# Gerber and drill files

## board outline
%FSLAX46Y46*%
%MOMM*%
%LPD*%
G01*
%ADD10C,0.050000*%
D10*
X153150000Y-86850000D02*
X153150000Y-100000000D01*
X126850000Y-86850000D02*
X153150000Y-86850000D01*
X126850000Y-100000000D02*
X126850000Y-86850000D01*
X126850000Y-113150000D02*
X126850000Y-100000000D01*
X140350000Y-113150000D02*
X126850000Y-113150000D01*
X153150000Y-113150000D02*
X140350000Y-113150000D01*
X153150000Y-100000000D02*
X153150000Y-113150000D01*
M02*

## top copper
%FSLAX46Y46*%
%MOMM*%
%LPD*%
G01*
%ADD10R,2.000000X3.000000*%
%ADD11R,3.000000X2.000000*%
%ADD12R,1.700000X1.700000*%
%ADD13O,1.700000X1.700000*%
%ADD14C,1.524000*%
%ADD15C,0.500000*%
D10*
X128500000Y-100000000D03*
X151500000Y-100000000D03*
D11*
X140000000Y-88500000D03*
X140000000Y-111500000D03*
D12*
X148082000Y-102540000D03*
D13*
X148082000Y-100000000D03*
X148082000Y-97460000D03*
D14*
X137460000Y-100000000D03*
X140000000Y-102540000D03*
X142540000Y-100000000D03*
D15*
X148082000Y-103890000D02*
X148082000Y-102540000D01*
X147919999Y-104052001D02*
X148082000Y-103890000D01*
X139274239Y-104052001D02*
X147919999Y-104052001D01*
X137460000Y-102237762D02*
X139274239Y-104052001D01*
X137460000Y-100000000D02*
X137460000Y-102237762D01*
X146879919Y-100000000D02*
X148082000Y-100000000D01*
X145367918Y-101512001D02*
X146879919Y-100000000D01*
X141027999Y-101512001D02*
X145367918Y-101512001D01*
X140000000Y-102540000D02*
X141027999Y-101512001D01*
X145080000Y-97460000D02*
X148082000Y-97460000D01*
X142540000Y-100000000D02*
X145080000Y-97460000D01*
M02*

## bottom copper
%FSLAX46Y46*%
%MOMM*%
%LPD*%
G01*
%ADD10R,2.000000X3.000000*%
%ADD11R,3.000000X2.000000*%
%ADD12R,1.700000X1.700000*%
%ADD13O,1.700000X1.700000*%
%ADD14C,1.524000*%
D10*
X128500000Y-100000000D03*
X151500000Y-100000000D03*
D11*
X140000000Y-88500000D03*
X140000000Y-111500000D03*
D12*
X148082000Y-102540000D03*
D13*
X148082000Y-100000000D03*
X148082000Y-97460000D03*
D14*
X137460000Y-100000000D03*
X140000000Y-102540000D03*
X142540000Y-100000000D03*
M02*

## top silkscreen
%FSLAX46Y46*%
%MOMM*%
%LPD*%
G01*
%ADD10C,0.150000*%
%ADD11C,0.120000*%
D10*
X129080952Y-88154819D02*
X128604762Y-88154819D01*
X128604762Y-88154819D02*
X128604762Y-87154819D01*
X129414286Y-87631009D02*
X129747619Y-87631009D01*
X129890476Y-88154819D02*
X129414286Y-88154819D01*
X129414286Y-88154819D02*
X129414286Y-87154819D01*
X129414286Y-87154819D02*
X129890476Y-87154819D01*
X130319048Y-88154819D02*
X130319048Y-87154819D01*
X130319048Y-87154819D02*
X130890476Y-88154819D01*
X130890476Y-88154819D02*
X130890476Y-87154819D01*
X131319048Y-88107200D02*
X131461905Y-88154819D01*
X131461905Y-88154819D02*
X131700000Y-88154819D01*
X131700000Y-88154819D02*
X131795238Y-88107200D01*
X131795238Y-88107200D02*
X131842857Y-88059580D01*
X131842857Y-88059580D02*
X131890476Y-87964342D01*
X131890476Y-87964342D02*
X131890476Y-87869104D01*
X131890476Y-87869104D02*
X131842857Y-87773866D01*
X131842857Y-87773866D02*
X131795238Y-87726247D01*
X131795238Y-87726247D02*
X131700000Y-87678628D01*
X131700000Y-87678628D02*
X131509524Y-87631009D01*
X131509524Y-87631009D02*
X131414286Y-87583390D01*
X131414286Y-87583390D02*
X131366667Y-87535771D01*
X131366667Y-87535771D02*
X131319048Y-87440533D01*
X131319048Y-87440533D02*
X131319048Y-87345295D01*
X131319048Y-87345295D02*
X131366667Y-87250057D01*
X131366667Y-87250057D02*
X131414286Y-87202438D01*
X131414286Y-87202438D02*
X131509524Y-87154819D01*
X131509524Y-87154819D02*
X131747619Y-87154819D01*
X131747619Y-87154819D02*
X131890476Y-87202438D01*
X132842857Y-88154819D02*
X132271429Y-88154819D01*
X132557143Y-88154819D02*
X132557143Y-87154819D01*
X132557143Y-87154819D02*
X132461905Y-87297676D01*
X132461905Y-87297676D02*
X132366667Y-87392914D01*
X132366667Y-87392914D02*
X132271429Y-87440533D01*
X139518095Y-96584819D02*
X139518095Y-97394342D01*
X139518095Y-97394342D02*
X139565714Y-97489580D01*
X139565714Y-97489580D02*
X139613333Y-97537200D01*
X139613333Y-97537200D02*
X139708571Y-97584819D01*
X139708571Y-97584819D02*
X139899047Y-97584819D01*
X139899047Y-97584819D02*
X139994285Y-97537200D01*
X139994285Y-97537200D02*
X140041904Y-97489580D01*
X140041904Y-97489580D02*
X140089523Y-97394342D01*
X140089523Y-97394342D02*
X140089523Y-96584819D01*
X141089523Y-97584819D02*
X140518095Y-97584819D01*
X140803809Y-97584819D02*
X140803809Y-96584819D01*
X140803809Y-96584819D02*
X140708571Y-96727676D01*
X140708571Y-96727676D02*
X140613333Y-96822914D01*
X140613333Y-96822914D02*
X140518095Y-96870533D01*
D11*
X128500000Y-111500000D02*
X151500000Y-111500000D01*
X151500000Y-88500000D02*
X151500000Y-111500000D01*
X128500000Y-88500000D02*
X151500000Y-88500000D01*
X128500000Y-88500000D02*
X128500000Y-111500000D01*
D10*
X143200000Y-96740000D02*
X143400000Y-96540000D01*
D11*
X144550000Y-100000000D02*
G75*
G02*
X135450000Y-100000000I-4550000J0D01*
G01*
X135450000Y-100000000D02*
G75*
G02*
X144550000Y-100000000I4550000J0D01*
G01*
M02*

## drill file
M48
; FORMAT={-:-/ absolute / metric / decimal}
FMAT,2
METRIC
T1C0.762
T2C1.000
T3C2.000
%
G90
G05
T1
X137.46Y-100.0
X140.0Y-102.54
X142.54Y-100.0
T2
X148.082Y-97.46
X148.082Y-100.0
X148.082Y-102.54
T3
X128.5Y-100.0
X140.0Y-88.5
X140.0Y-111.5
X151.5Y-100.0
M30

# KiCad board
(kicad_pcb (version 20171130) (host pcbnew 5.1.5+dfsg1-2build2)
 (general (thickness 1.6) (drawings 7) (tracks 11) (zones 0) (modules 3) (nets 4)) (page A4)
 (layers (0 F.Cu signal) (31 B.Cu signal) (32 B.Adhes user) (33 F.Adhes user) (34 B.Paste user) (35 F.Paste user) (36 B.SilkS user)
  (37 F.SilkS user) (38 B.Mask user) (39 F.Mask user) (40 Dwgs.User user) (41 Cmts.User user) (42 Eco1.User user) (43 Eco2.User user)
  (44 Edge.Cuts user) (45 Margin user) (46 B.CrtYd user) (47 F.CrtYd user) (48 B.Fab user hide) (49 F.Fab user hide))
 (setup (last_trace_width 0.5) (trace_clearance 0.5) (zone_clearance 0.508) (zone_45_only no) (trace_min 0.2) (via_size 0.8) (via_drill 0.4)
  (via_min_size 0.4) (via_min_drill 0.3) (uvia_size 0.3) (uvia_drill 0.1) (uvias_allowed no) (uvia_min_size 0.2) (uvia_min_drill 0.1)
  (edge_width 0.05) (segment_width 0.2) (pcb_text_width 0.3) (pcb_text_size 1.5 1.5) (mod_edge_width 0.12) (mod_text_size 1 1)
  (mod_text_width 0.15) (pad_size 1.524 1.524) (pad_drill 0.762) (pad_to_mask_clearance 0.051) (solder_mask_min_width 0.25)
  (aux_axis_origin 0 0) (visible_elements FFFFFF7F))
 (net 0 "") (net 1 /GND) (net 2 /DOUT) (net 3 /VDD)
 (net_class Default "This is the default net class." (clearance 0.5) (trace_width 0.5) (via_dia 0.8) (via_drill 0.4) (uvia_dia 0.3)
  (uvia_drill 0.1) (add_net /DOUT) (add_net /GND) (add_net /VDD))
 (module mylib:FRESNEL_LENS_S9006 (layer F.Cu) (at 140 100)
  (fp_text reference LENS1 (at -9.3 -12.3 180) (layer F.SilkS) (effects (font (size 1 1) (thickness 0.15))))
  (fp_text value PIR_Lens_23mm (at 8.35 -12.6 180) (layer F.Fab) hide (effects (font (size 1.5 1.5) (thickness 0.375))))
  (fp_line (start -11.5 11.5) (end 11.5 11.5) (layer F.SilkS) (width 0.12))
  (fp_line (start 11.5 -11.5) (end 11.5 11.5) (layer F.SilkS) (width 0.12))
  (fp_line (start -11.5 -11.5) (end 11.5 -11.5) (layer F.SilkS) (width 0.12))
  (fp_line (start -11.5 -11.5) (end -11.5 11.5) (layer F.SilkS) (width 0.12))
  (pad "" np_thru_hole rect (at -11.5 0) (size 2 3) (drill 2) (layers *.Cu *.Mask) (clearance 0.5))
  (pad "" np_thru_hole rect (at 11.5 0) (size 2 3) (drill 2) (layers *.Cu *.Mask) (clearance 0.5))
  (pad "" np_thru_hole rect (at 0 -11.5 90) (size 2 3) (drill 2) (layers *.Cu *.Mask) (clearance 0.5))
  (pad "" np_thru_hole rect (at 0 11.5 90) (size 2 3) (drill 2) (layers *.Cu *.Mask) (clearance 0.5)))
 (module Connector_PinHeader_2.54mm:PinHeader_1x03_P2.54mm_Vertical (layer B.Cu) (at 148.082 102.54)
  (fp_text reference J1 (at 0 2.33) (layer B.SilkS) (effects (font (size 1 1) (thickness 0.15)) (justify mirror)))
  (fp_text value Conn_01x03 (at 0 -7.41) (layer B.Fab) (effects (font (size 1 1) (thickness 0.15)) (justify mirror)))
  (pad 1 thru_hole rect (at 0 0) (size 1.7 1.7) (drill 1) (layers *.Cu *.Mask) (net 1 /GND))
  (pad 2 thru_hole oval (at 0 -2.54) (size 1.7 1.7) (drill 1) (layers *.Cu *.Mask) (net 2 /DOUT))
  (pad 3 thru_hole oval (at 0 -5.08) (size 1.7 1.7) (drill 1) (layers *.Cu *.Mask) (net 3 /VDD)))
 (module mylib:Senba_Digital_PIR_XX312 (layer F.Cu) (at 140 100)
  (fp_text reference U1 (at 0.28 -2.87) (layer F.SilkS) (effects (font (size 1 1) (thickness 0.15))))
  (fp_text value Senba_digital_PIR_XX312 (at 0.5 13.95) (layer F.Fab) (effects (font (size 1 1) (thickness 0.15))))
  (fp_line (start 3.2 -3.26) (end 3.4 -3.46) (layer F.SilkS) (width 0.15))
  (fp_circle (center 0 0) (end 4.55 0) (layer F.SilkS) (width 0.12))
  (pad 3 thru_hole circle (at -2.54 0) (size 1.524 1.524) (drill 0.762) (layers *.Cu *.Mask) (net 1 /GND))
  (pad 2 thru_hole circle (at 0 2.54) (size 1.524 1.524) (drill 0.762) (layers *.Cu *.Mask) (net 2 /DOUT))
  (pad 1 thru_hole circle (at 2.54 0) (size 1.524 1.524) (drill 0.762) (layers *.Cu *.Mask) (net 3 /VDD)))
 (gr_line (start 153.15 86.85) (end 153.15 100) (layer Edge.Cuts) (width 0.05))
 (gr_line (start 126.85 86.85) (end 153.15 86.85) (layer Edge.Cuts) (width 0.05))
 (gr_line (start 126.85 100) (end 126.85 86.85) (layer Edge.Cuts) (width 0.05))
 (gr_line (start 126.85 113.15) (end 126.85 100) (layer Edge.Cuts) (width 0.05))
 (gr_line (start 140.35 113.15) (end 126.85 113.15) (layer Edge.Cuts) (width 0.05))
 (gr_line (start 153.15 113.15) (end 140.35 113.15) (layer Edge.Cuts) (width 0.05))
 (gr_line (start 153.15 100) (end 153.15 113.15) (layer Edge.Cuts) (width 0.05))
 (segment (start 148.082 103.89) (end 148.082 102.54) (width 0.5) (layer F.Cu) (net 1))
 (segment (start 147.919999 104.052001) (end 148.082 103.89) (width 0.5) (layer F.Cu) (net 1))
 (segment (start 139.274239 104.052001) (end 147.919999 104.052001) (width 0.5) (layer F.Cu) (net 1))
 (segment (start 137.46 102.237762) (end 139.274239 104.052001) (width 0.5) (layer F.Cu) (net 1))
 (segment (start 137.46 100) (end 137.46 102.237762) (width 0.5) (layer F.Cu) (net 1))
 (segment (start 146.879919 100) (end 148.082 100) (width 0.5) (layer F.Cu) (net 2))
 (segment (start 145.367918 101.512001) (end 146.879919 100) (width 0.5) (layer F.Cu) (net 2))
 (segment (start 141.027999 101.512001) (end 145.367918 101.512001) (width 0.5) (layer F.Cu) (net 2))
 (segment (start 140 102.54) (end 141.027999 101.512001) (width 0.5) (layer F.Cu) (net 2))
 (segment (start 145.08 97.46) (end 148.082 97.46) (width 0.5) (layer F.Cu) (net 3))
 (segment (start 142.54 100) (end 145.08 97.46) (width 0.5) (layer F.Cu) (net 3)))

